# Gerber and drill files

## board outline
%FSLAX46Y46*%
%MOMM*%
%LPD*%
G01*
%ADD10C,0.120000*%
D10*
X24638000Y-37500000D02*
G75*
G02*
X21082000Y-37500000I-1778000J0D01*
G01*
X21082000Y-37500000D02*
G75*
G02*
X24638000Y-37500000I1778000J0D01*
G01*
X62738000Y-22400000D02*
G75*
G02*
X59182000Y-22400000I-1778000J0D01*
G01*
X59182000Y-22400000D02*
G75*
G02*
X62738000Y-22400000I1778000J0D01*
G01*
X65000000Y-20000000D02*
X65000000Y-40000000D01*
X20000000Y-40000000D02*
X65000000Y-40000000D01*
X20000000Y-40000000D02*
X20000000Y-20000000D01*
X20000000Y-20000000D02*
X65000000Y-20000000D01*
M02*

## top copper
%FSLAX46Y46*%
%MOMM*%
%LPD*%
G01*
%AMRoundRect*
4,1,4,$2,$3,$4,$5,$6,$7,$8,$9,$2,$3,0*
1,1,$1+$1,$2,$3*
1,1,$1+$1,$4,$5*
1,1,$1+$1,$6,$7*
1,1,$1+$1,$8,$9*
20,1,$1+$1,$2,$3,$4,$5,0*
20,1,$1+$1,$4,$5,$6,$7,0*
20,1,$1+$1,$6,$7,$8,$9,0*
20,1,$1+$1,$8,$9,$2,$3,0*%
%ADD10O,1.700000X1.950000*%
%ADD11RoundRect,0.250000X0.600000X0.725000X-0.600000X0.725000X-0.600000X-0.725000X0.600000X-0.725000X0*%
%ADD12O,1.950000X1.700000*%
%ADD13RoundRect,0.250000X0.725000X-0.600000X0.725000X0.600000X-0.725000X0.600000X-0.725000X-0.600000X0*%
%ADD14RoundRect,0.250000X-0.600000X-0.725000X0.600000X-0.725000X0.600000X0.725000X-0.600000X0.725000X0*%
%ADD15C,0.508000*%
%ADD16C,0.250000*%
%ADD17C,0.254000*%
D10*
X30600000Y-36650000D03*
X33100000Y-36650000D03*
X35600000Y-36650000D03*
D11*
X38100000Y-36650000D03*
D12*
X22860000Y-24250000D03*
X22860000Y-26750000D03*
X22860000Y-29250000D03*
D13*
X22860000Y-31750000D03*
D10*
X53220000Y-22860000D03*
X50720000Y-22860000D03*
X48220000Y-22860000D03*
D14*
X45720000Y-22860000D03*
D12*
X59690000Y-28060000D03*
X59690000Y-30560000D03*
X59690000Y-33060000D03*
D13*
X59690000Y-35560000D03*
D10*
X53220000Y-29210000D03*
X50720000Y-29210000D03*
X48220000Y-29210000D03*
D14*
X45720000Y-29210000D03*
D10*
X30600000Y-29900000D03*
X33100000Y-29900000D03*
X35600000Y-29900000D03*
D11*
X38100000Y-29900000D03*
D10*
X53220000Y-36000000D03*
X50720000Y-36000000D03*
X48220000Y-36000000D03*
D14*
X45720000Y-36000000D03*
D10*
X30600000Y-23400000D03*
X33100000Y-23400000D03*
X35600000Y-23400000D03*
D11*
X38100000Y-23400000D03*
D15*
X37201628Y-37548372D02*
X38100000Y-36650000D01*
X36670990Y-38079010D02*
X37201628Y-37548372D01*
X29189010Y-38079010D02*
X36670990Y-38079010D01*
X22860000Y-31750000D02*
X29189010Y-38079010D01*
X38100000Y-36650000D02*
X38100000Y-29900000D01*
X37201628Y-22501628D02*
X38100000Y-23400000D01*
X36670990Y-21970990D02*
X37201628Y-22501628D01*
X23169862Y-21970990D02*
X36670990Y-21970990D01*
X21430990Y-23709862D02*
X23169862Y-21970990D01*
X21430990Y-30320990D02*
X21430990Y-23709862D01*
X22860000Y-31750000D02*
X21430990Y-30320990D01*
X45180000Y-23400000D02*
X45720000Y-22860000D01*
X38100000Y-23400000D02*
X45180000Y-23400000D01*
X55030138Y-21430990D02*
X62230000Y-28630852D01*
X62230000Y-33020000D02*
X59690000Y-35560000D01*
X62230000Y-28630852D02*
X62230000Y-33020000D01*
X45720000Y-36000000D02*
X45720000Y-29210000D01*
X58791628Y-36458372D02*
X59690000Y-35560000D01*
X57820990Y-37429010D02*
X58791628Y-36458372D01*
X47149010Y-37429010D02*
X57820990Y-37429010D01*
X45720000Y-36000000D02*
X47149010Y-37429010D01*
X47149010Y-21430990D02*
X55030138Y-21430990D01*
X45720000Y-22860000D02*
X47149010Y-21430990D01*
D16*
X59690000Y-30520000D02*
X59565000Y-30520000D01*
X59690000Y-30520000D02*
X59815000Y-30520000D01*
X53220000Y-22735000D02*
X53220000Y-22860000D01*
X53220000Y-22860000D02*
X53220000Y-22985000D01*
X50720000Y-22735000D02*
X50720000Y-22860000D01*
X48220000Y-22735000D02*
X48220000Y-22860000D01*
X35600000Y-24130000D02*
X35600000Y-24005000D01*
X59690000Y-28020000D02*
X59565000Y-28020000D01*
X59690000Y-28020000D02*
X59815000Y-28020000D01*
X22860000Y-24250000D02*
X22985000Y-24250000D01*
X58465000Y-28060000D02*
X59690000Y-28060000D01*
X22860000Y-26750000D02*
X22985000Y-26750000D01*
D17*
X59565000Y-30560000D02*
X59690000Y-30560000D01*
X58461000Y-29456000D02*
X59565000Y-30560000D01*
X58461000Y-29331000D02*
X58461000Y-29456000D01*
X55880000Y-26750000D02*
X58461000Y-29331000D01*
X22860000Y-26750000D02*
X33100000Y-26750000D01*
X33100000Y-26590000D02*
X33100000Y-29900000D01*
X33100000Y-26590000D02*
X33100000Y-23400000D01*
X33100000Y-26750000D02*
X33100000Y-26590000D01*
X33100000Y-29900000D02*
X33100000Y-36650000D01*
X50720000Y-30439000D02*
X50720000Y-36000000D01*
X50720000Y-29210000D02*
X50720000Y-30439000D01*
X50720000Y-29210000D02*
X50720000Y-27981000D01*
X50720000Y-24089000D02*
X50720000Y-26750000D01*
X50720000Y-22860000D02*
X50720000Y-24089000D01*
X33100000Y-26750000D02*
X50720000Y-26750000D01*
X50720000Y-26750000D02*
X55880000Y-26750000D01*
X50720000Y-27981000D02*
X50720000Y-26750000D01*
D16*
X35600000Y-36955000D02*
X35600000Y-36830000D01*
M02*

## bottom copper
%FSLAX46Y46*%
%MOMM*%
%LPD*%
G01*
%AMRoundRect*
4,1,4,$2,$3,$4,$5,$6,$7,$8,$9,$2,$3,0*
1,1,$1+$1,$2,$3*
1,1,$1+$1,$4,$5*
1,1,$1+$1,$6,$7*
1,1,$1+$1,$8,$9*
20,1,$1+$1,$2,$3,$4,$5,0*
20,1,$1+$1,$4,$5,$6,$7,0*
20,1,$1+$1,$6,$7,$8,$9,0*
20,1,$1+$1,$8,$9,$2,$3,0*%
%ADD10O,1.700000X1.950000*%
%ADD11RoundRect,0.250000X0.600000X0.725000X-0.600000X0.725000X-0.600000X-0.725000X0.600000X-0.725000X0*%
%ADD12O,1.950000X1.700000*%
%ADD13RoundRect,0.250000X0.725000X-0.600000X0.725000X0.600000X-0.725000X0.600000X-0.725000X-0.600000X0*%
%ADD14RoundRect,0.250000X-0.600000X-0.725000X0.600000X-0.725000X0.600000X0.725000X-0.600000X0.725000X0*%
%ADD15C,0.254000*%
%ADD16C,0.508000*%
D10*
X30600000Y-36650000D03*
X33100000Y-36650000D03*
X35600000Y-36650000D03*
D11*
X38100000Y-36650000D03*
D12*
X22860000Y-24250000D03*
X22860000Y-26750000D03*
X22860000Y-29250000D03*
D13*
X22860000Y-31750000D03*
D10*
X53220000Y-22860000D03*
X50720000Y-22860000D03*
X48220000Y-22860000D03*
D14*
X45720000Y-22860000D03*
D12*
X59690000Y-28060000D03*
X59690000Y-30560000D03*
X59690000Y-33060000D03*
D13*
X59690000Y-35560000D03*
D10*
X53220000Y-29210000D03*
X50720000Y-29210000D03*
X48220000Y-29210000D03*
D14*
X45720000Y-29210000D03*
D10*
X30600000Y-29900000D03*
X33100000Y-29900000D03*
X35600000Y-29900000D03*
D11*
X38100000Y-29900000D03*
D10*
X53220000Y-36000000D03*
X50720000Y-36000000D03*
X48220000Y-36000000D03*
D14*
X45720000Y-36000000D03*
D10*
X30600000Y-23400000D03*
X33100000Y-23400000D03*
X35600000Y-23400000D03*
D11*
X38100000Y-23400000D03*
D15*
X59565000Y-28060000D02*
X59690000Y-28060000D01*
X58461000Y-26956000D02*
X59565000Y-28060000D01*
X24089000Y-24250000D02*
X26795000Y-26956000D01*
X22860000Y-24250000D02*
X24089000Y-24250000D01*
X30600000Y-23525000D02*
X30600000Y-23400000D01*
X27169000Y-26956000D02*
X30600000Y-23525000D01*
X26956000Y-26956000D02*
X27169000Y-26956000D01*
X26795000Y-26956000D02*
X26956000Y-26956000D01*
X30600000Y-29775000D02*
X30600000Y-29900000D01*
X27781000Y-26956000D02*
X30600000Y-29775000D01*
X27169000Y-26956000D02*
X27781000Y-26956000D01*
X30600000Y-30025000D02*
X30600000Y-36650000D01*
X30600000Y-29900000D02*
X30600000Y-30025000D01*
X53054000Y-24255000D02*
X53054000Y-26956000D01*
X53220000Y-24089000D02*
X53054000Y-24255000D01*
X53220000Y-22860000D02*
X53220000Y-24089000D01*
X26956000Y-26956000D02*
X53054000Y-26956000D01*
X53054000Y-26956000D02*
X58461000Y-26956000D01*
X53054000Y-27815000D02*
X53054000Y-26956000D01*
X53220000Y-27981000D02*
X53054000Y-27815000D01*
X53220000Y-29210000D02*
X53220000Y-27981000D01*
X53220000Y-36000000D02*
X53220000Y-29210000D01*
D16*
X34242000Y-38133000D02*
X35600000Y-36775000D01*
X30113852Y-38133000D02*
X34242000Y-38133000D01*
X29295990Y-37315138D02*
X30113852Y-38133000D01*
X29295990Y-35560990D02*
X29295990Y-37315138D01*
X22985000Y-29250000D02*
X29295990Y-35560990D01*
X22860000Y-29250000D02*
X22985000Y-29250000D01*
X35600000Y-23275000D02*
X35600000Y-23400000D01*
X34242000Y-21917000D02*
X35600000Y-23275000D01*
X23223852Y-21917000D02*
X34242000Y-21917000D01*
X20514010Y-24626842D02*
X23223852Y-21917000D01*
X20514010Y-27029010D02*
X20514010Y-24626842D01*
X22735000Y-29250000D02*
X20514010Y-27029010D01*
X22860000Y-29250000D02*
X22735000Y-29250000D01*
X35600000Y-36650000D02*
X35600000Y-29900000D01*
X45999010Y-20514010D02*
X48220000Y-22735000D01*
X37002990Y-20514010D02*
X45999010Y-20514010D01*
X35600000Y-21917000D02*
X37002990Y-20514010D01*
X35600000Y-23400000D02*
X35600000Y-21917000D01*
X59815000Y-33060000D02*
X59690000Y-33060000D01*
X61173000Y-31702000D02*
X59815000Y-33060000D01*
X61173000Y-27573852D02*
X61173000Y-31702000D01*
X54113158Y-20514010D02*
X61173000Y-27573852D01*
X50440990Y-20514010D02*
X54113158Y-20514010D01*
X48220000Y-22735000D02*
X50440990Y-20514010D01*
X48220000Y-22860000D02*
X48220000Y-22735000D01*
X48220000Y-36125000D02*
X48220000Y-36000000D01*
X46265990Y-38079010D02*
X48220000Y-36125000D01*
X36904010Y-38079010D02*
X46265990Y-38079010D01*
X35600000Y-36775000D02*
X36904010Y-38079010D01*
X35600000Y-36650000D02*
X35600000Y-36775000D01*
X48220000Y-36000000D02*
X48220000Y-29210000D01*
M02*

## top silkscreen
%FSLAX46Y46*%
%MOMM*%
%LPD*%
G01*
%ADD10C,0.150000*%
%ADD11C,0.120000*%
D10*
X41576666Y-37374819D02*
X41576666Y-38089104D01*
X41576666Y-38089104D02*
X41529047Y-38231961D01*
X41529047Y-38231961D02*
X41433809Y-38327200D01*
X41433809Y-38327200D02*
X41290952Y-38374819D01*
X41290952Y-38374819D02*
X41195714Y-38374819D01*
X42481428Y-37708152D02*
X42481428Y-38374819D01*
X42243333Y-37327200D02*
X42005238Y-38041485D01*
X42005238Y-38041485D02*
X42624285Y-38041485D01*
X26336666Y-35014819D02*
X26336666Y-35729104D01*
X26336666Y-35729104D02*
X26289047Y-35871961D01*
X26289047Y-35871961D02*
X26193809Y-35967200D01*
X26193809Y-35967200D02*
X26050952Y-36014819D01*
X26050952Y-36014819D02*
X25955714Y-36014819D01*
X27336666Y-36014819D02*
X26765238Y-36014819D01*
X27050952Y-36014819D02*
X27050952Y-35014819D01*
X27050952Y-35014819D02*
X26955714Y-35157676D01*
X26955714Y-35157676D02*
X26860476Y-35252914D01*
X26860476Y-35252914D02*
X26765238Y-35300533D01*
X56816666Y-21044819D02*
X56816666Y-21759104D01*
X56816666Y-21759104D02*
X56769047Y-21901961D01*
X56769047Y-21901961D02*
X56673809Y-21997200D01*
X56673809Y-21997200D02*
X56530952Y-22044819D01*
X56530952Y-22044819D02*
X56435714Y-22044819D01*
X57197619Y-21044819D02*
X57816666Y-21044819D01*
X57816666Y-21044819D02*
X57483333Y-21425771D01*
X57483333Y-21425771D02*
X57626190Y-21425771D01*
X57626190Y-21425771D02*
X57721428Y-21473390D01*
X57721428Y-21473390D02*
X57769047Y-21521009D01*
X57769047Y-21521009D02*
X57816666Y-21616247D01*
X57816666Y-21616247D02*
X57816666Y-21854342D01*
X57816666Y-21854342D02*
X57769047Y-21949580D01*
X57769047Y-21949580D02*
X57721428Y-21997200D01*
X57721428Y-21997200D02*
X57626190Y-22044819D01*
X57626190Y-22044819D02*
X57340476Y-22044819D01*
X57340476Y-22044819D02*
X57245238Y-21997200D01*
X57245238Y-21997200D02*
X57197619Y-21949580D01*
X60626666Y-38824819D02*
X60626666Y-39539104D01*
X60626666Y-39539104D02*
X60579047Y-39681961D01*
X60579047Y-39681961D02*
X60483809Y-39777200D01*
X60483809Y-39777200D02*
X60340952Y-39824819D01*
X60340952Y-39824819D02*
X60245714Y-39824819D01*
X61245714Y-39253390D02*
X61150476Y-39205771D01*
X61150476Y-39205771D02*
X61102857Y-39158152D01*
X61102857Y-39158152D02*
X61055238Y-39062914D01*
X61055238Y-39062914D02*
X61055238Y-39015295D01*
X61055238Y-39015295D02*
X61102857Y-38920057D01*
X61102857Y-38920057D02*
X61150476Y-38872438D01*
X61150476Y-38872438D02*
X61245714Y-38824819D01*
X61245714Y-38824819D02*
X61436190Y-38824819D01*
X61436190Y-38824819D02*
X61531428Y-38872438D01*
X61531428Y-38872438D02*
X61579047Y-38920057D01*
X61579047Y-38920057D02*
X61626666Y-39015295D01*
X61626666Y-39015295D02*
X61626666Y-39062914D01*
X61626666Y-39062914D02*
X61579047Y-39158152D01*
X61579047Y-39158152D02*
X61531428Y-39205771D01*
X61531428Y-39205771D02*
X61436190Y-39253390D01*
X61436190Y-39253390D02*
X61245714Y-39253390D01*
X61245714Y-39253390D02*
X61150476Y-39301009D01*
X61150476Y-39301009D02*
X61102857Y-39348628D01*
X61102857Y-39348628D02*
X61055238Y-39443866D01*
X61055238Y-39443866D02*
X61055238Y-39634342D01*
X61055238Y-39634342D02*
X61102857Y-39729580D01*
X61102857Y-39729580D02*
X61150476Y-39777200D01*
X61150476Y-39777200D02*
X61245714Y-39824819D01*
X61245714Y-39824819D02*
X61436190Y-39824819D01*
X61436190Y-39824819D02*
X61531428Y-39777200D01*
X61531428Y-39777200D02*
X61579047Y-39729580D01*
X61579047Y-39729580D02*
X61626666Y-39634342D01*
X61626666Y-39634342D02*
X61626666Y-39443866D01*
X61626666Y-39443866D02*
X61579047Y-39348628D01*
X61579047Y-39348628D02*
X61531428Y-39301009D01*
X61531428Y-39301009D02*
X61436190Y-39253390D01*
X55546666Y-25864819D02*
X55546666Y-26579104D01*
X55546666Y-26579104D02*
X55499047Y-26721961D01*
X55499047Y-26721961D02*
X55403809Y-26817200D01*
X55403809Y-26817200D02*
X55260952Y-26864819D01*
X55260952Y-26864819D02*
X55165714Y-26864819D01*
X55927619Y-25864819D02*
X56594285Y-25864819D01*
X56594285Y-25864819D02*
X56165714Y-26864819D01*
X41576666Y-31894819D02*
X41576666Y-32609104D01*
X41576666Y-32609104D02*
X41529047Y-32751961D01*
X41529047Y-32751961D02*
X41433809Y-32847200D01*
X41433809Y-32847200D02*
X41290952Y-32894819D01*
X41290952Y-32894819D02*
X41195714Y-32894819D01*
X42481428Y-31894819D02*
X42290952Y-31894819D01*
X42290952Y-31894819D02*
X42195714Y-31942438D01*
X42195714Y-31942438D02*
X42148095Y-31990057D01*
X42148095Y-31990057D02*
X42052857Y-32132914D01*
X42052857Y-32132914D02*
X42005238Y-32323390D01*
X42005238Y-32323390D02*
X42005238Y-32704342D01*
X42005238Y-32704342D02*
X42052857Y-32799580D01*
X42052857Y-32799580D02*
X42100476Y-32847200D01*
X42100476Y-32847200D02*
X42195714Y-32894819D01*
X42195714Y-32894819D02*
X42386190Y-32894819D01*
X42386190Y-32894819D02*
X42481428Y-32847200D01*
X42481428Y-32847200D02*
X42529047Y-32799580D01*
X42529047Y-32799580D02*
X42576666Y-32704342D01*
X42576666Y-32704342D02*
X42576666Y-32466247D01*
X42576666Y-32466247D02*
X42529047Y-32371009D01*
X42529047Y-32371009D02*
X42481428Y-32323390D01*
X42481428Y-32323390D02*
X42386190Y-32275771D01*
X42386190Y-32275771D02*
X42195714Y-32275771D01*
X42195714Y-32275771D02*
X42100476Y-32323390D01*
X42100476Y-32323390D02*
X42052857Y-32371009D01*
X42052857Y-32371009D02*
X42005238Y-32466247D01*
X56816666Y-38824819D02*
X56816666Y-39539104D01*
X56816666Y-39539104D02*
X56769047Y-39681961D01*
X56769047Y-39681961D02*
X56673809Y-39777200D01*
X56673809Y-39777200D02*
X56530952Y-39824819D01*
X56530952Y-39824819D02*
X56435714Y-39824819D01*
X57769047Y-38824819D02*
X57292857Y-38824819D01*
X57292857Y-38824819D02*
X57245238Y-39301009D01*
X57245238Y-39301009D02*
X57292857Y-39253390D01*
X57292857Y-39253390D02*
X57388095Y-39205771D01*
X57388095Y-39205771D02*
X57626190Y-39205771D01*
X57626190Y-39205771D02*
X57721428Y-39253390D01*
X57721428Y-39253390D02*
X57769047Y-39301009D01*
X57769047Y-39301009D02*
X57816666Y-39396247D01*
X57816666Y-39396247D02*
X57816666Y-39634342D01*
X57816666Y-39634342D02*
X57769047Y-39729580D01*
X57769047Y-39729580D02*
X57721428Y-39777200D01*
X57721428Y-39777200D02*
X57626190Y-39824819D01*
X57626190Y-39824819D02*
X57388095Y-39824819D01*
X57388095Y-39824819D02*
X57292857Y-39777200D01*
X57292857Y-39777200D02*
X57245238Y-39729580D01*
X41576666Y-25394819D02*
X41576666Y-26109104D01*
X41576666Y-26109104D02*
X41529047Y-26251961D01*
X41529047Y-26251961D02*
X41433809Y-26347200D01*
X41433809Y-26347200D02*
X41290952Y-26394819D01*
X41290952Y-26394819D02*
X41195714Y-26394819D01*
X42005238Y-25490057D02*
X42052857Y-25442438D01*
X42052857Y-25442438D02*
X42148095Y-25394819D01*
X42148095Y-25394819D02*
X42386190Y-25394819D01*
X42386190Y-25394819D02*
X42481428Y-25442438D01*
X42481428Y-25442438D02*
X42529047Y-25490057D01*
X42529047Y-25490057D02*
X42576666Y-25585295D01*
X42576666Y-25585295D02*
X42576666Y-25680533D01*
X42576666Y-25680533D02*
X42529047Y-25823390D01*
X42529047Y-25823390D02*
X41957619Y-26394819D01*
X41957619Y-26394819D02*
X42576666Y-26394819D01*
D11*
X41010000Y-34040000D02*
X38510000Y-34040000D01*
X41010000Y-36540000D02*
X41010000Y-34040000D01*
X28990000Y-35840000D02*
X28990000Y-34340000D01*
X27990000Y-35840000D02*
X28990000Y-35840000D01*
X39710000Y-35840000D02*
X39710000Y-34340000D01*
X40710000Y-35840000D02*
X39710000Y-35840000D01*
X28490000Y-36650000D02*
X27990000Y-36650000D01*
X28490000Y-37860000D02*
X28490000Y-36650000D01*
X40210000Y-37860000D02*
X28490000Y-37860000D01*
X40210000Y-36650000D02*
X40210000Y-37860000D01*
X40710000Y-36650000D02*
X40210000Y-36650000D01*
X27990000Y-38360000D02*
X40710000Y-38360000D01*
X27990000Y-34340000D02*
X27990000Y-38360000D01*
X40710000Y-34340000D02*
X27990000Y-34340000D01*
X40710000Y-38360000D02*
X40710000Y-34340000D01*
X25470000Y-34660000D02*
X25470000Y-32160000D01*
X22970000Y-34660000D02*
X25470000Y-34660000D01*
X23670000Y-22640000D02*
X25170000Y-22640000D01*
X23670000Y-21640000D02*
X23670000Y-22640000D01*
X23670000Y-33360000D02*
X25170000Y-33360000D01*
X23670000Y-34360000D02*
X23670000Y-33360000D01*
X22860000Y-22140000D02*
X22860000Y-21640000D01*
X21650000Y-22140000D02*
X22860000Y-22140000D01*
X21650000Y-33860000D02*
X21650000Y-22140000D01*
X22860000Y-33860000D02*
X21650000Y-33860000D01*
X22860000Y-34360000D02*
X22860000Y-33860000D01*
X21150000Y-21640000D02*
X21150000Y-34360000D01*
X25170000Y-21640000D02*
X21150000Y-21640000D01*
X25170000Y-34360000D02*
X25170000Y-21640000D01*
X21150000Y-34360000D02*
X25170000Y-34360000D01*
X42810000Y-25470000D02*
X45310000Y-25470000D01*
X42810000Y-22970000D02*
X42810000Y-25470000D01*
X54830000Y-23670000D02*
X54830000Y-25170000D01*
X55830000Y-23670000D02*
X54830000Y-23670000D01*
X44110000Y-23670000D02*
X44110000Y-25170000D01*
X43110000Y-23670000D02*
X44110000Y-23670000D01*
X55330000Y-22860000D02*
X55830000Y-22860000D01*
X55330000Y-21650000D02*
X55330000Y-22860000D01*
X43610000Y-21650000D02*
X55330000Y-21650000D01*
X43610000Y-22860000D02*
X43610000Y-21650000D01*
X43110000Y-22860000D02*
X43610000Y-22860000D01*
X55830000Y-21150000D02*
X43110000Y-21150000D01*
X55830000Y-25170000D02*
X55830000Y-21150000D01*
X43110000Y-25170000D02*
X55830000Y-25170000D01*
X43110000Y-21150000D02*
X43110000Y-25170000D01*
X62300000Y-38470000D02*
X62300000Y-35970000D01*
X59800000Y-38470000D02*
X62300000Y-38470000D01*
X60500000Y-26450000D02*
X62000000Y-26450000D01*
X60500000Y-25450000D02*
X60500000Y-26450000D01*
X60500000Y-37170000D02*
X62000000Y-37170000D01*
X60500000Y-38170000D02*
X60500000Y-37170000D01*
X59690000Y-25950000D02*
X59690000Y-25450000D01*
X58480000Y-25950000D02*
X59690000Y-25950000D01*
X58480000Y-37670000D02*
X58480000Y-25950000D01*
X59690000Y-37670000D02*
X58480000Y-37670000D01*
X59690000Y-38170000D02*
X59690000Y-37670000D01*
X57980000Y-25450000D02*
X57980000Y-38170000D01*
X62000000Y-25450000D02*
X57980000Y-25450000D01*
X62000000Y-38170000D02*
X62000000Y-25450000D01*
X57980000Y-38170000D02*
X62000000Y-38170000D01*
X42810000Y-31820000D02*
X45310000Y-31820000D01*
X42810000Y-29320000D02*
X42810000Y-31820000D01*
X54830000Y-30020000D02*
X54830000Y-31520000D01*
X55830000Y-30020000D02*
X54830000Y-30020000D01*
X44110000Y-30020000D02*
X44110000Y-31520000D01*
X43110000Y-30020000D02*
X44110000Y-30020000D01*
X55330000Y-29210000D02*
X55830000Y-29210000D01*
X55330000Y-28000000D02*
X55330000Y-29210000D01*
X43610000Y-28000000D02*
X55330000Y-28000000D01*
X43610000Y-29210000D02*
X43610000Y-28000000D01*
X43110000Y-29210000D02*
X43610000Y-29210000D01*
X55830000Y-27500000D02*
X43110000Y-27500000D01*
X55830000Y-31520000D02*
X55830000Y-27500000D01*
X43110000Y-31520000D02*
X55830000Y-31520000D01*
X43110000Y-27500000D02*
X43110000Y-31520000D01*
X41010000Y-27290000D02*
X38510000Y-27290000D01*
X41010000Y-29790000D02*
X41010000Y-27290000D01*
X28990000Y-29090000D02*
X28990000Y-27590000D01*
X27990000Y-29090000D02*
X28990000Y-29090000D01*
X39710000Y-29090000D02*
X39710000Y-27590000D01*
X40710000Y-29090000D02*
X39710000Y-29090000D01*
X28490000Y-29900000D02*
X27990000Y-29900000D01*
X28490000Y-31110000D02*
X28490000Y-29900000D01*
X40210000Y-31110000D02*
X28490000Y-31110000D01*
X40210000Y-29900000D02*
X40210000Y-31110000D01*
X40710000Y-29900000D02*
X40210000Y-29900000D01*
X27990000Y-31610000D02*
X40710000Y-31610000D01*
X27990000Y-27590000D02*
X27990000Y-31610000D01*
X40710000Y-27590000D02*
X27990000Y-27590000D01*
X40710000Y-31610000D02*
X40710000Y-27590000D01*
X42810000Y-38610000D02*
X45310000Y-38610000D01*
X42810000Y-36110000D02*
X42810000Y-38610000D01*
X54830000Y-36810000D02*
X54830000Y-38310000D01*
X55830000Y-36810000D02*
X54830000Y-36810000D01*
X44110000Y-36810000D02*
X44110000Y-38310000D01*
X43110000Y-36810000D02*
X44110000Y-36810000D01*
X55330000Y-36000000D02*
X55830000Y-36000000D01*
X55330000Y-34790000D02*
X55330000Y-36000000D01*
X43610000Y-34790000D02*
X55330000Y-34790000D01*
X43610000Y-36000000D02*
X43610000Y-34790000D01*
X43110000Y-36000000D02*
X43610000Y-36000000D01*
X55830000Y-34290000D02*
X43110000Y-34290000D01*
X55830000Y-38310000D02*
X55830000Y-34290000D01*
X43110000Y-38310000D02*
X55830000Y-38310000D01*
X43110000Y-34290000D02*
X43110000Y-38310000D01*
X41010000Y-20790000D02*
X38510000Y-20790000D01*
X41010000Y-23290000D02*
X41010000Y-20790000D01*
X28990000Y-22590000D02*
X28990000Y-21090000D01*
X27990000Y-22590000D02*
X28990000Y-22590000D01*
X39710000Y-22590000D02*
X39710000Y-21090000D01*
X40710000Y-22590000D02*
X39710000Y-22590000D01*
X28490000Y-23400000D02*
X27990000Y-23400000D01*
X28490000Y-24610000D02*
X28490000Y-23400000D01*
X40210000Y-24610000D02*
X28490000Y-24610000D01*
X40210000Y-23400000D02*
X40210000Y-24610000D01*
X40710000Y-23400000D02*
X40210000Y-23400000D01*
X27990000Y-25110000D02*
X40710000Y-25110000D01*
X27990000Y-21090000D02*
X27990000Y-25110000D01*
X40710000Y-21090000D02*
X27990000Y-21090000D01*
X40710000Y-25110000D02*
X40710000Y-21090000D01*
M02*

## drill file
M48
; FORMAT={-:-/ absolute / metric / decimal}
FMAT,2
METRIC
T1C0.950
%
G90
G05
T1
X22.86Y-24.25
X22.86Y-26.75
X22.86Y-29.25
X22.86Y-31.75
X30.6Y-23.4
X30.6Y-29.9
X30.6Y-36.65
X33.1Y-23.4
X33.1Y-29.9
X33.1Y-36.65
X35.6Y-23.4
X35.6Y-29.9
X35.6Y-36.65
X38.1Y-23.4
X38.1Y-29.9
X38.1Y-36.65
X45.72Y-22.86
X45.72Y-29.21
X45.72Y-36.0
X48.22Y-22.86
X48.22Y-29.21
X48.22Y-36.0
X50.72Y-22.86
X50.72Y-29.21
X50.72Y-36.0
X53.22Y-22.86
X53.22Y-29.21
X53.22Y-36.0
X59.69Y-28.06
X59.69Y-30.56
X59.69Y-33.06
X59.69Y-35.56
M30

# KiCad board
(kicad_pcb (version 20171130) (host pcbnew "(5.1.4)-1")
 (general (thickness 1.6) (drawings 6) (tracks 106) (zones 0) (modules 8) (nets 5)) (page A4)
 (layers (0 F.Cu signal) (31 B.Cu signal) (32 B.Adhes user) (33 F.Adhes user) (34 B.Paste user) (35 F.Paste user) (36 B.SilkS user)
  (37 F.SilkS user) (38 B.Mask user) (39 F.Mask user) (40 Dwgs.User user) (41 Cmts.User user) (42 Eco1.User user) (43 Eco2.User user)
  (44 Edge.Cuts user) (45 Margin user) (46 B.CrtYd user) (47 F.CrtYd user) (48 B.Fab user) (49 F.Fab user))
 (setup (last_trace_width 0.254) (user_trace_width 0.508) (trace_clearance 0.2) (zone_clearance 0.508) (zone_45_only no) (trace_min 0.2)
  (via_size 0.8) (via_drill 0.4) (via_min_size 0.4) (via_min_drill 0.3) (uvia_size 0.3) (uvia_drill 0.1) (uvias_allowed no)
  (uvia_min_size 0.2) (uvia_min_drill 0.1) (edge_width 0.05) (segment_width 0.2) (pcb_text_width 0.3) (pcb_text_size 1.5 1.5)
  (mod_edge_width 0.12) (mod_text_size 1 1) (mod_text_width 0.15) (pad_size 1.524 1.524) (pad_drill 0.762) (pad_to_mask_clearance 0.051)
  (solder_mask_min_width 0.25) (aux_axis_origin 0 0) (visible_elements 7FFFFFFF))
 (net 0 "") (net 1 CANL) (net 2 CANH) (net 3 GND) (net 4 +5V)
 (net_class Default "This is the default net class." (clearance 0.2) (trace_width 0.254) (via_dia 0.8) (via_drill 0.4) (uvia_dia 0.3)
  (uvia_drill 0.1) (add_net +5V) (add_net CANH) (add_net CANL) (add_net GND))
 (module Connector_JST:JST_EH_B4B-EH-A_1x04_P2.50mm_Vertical (layer F.Cu) (at 38.1 36.65 180)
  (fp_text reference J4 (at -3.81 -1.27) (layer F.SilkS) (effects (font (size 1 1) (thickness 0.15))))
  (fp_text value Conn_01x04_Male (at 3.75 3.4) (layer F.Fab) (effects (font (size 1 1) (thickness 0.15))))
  (fp_line (start -2.91 2.61) (end -0.41 2.61) (layer F.SilkS) (width 0.12))
  (fp_line (start -2.91 0.11) (end -2.91 2.61) (layer F.SilkS) (width 0.12))
  (fp_line (start 9.11 0.81) (end 9.11 2.31) (layer F.SilkS) (width 0.12))
  (fp_line (start 10.11 0.81) (end 9.11 0.81) (layer F.SilkS) (width 0.12))
  (fp_line (start -1.61 0.81) (end -1.61 2.31) (layer F.SilkS) (width 0.12))
  (fp_line (start -2.61 0.81) (end -1.61 0.81) (layer F.SilkS) (width 0.12))
  (fp_line (start 9.61 0) (end 10.11 0) (layer F.SilkS) (width 0.12))
  (fp_line (start 9.61 -1.21) (end 9.61 0) (layer F.SilkS) (width 0.12))
  (fp_line (start -2.11 -1.21) (end 9.61 -1.21) (layer F.SilkS) (width 0.12))
  (fp_line (start -2.11 0) (end -2.11 -1.21) (layer F.SilkS) (width 0.12))
  (fp_line (start -2.61 0) (end -2.11 0) (layer F.SilkS) (width 0.12))
  (fp_line (start 10.11 -1.71) (end -2.61 -1.71) (layer F.SilkS) (width 0.12))
  (fp_line (start 10.11 2.31) (end 10.11 -1.71) (layer F.SilkS) (width 0.12))
  (fp_line (start -2.61 2.31) (end 10.11 2.31) (layer F.SilkS) (width 0.12))
  (fp_line (start -2.61 -1.71) (end -2.61 2.31) (layer F.SilkS) (width 0.12))
  (pad 4 thru_hole oval (at 7.5 0 180) (size 1.7 1.95) (drill 0.95) (layers *.Cu *.Mask) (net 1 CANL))
  (pad 3 thru_hole oval (at 5 0 180) (size 1.7 1.95) (drill 0.95) (layers *.Cu *.Mask) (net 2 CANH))
  (pad 2 thru_hole oval (at 2.5 0 180) (size 1.7 1.95) (drill 0.95) (layers *.Cu *.Mask) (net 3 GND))
  (pad 1 thru_hole roundrect (at 0 0 180) (size 1.7 1.95) (drill 0.95) (layers *.Cu *.Mask) (roundrect_rratio 0.147059) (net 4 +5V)))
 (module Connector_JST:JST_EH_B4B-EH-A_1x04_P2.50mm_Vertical (layer F.Cu) (at 22.86 31.75 90)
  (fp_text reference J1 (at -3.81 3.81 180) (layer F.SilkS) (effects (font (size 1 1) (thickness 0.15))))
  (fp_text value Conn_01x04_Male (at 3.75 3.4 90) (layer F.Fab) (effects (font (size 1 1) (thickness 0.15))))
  (fp_line (start -2.91 2.61) (end -0.41 2.61) (layer F.SilkS) (width 0.12))
  (fp_line (start -2.91 0.11) (end -2.91 2.61) (layer F.SilkS) (width 0.12))
  (fp_line (start 9.11 0.81) (end 9.11 2.31) (layer F.SilkS) (width 0.12))
  (fp_line (start 10.11 0.81) (end 9.11 0.81) (layer F.SilkS) (width 0.12))
  (fp_line (start -1.61 0.81) (end -1.61 2.31) (layer F.SilkS) (width 0.12))
  (fp_line (start -2.61 0.81) (end -1.61 0.81) (layer F.SilkS) (width 0.12))
  (fp_line (start 9.61 0) (end 10.11 0) (layer F.SilkS) (width 0.12))
  (fp_line (start 9.61 -1.21) (end 9.61 0) (layer F.SilkS) (width 0.12))
  (fp_line (start -2.11 -1.21) (end 9.61 -1.21) (layer F.SilkS) (width 0.12))
  (fp_line (start -2.11 0) (end -2.11 -1.21) (layer F.SilkS) (width 0.12))
  (fp_line (start -2.61 0) (end -2.11 0) (layer F.SilkS) (width 0.12))
  (fp_line (start 10.11 -1.71) (end -2.61 -1.71) (layer F.SilkS) (width 0.12))
  (fp_line (start 10.11 2.31) (end 10.11 -1.71) (layer F.SilkS) (width 0.12))
  (fp_line (start -2.61 2.31) (end 10.11 2.31) (layer F.SilkS) (width 0.12))
  (fp_line (start -2.61 -1.71) (end -2.61 2.31) (layer F.SilkS) (width 0.12))
  (pad 4 thru_hole oval (at 7.5 0 90) (size 1.7 1.95) (drill 0.95) (layers *.Cu *.Mask) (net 1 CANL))
  (pad 3 thru_hole oval (at 5 0 90) (size 1.7 1.95) (drill 0.95) (layers *.Cu *.Mask) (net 2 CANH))
  (pad 2 thru_hole oval (at 2.5 0 90) (size 1.7 1.95) (drill 0.95) (layers *.Cu *.Mask) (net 3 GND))
  (pad 1 thru_hole roundrect (at 0 0 90) (size 1.7 1.95) (drill 0.95) (layers *.Cu *.Mask) (roundrect_rratio 0.147059) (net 4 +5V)))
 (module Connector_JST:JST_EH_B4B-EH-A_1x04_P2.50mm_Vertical (layer F.Cu) (at 45.72 22.86)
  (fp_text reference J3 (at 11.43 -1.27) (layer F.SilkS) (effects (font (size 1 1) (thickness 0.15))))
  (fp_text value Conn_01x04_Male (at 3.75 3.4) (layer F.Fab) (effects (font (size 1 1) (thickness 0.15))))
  (fp_line (start -2.91 2.61) (end -0.41 2.61) (layer F.SilkS) (width 0.12))
  (fp_line (start -2.91 0.11) (end -2.91 2.61) (layer F.SilkS) (width 0.12))
  (fp_line (start 9.11 0.81) (end 9.11 2.31) (layer F.SilkS) (width 0.12))
  (fp_line (start 10.11 0.81) (end 9.11 0.81) (layer F.SilkS) (width 0.12))
  (fp_line (start -1.61 0.81) (end -1.61 2.31) (layer F.SilkS) (width 0.12))
  (fp_line (start -2.61 0.81) (end -1.61 0.81) (layer F.SilkS) (width 0.12))
  (fp_line (start 9.61 0) (end 10.11 0) (layer F.SilkS) (width 0.12))
  (fp_line (start 9.61 -1.21) (end 9.61 0) (layer F.SilkS) (width 0.12))
  (fp_line (start -2.11 -1.21) (end 9.61 -1.21) (layer F.SilkS) (width 0.12))
  (fp_line (start -2.11 0) (end -2.11 -1.21) (layer F.SilkS) (width 0.12))
  (fp_line (start -2.61 0) (end -2.11 0) (layer F.SilkS) (width 0.12))
  (fp_line (start 10.11 -1.71) (end -2.61 -1.71) (layer F.SilkS) (width 0.12))
  (fp_line (start 10.11 2.31) (end 10.11 -1.71) (layer F.SilkS) (width 0.12))
  (fp_line (start -2.61 2.31) (end 10.11 2.31) (layer F.SilkS) (width 0.12))
  (fp_line (start -2.61 -1.71) (end -2.61 2.31) (layer F.SilkS) (width 0.12))
  (pad 4 thru_hole oval (at 7.5 0) (size 1.7 1.95) (drill 0.95) (layers *.Cu *.Mask) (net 1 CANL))
  (pad 3 thru_hole oval (at 5 0) (size 1.7 1.95) (drill 0.95) (layers *.Cu *.Mask) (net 2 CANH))
  (pad 2 thru_hole oval (at 2.5 0) (size 1.7 1.95) (drill 0.95) (layers *.Cu *.Mask) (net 3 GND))
  (pad 1 thru_hole roundrect (at 0 0) (size 1.7 1.95) (drill 0.95) (layers *.Cu *.Mask) (roundrect_rratio 0.147059) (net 4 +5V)))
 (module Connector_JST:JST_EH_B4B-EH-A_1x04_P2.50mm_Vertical (layer F.Cu) (at 59.69 35.56 90)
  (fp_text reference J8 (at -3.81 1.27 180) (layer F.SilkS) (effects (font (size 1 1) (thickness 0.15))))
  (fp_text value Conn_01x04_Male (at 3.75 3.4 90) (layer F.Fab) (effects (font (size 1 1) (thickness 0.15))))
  (fp_line (start -2.91 2.61) (end -0.41 2.61) (layer F.SilkS) (width 0.12))
  (fp_line (start -2.91 0.11) (end -2.91 2.61) (layer F.SilkS) (width 0.12))
  (fp_line (start 9.11 0.81) (end 9.11 2.31) (layer F.SilkS) (width 0.12))
  (fp_line (start 10.11 0.81) (end 9.11 0.81) (layer F.SilkS) (width 0.12))
  (fp_line (start -1.61 0.81) (end -1.61 2.31) (layer F.SilkS) (width 0.12))
  (fp_line (start -2.61 0.81) (end -1.61 0.81) (layer F.SilkS) (width 0.12))
  (fp_line (start 9.61 0) (end 10.11 0) (layer F.SilkS) (width 0.12))
  (fp_line (start 9.61 -1.21) (end 9.61 0) (layer F.SilkS) (width 0.12))
  (fp_line (start -2.11 -1.21) (end 9.61 -1.21) (layer F.SilkS) (width 0.12))
  (fp_line (start -2.11 0) (end -2.11 -1.21) (layer F.SilkS) (width 0.12))
  (fp_line (start -2.61 0) (end -2.11 0) (layer F.SilkS) (width 0.12))
  (fp_line (start 10.11 -1.71) (end -2.61 -1.71) (layer F.SilkS) (width 0.12))
  (fp_line (start 10.11 2.31) (end 10.11 -1.71) (layer F.SilkS) (width 0.12))
  (fp_line (start -2.61 2.31) (end 10.11 2.31) (layer F.SilkS) (width 0.12))
  (fp_line (start -2.61 -1.71) (end -2.61 2.31) (layer F.SilkS) (width 0.12))
  (pad 4 thru_hole oval (at 7.5 0 90) (size 1.7 1.95) (drill 0.95) (layers *.Cu *.Mask) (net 1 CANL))
  (pad 3 thru_hole oval (at 5 0 90) (size 1.7 1.95) (drill 0.95) (layers *.Cu *.Mask) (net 2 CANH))
  (pad 2 thru_hole oval (at 2.5 0 90) (size 1.7 1.95) (drill 0.95) (layers *.Cu *.Mask) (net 3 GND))
  (pad 1 thru_hole roundrect (at 0 0 90) (size 1.7 1.95) (drill 0.95) (layers *.Cu *.Mask) (roundrect_rratio 0.147059) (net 4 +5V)))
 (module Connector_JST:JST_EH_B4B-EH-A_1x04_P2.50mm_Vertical (layer F.Cu) (at 45.72 29.21)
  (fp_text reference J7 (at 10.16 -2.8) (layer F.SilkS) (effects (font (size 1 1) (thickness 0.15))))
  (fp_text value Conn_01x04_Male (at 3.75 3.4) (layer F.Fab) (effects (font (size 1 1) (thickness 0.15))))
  (fp_line (start -2.91 2.61) (end -0.41 2.61) (layer F.SilkS) (width 0.12))
  (fp_line (start -2.91 0.11) (end -2.91 2.61) (layer F.SilkS) (width 0.12))
  (fp_line (start 9.11 0.81) (end 9.11 2.31) (layer F.SilkS) (width 0.12))
  (fp_line (start 10.11 0.81) (end 9.11 0.81) (layer F.SilkS) (width 0.12))
  (fp_line (start -1.61 0.81) (end -1.61 2.31) (layer F.SilkS) (width 0.12))
  (fp_line (start -2.61 0.81) (end -1.61 0.81) (layer F.SilkS) (width 0.12))
  (fp_line (start 9.61 0) (end 10.11 0) (layer F.SilkS) (width 0.12))
  (fp_line (start 9.61 -1.21) (end 9.61 0) (layer F.SilkS) (width 0.12))
  (fp_line (start -2.11 -1.21) (end 9.61 -1.21) (layer F.SilkS) (width 0.12))
  (fp_line (start -2.11 0) (end -2.11 -1.21) (layer F.SilkS) (width 0.12))
  (fp_line (start -2.61 0) (end -2.11 0) (layer F.SilkS) (width 0.12))
  (fp_line (start 10.11 -1.71) (end -2.61 -1.71) (layer F.SilkS) (width 0.12))
  (fp_line (start 10.11 2.31) (end 10.11 -1.71) (layer F.SilkS) (width 0.12))
  (fp_line (start -2.61 2.31) (end 10.11 2.31) (layer F.SilkS) (width 0.12))
  (fp_line (start -2.61 -1.71) (end -2.61 2.31) (layer F.SilkS) (width 0.12))
  (pad 4 thru_hole oval (at 7.5 0) (size 1.7 1.95) (drill 0.95) (layers *.Cu *.Mask) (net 1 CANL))
  (pad 3 thru_hole oval (at 5 0) (size 1.7 1.95) (drill 0.95) (layers *.Cu *.Mask) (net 2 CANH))
  (pad 2 thru_hole oval (at 2.5 0) (size 1.7 1.95) (drill 0.95) (layers *.Cu *.Mask) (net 3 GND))
  (pad 1 thru_hole roundrect (at 0 0) (size 1.7 1.95) (drill 0.95) (layers *.Cu *.Mask) (roundrect_rratio 0.147059) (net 4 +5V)))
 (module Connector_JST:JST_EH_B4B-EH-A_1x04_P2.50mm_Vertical (layer F.Cu) (at 38.1 29.9 180)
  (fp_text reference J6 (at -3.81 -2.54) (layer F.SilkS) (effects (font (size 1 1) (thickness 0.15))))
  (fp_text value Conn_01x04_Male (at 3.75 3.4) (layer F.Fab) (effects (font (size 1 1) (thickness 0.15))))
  (fp_line (start -2.91 2.61) (end -0.41 2.61) (layer F.SilkS) (width 0.12))
  (fp_line (start -2.91 0.11) (end -2.91 2.61) (layer F.SilkS) (width 0.12))
  (fp_line (start 9.11 0.81) (end 9.11 2.31) (layer F.SilkS) (width 0.12))
  (fp_line (start 10.11 0.81) (end 9.11 0.81) (layer F.SilkS) (width 0.12))
  (fp_line (start -1.61 0.81) (end -1.61 2.31) (layer F.SilkS) (width 0.12))
  (fp_line (start -2.61 0.81) (end -1.61 0.81) (layer F.SilkS) (width 0.12))
  (fp_line (start 9.61 0) (end 10.11 0) (layer F.SilkS) (width 0.12))
  (fp_line (start 9.61 -1.21) (end 9.61 0) (layer F.SilkS) (width 0.12))
  (fp_line (start -2.11 -1.21) (end 9.61 -1.21) (layer F.SilkS) (width 0.12))
  (fp_line (start -2.11 0) (end -2.11 -1.21) (layer F.SilkS) (width 0.12))
  (fp_line (start -2.61 0) (end -2.11 0) (layer F.SilkS) (width 0.12))
  (fp_line (start 10.11 -1.71) (end -2.61 -1.71) (layer F.SilkS) (width 0.12))
  (fp_line (start 10.11 2.31) (end 10.11 -1.71) (layer F.SilkS) (width 0.12))
  (fp_line (start -2.61 2.31) (end 10.11 2.31) (layer F.SilkS) (width 0.12))
  (fp_line (start -2.61 -1.71) (end -2.61 2.31) (layer F.SilkS) (width 0.12))
  (pad 4 thru_hole oval (at 7.5 0 180) (size 1.7 1.95) (drill 0.95) (layers *.Cu *.Mask) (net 1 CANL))
  (pad 3 thru_hole oval (at 5 0 180) (size 1.7 1.95) (drill 0.95) (layers *.Cu *.Mask) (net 2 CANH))
  (pad 2 thru_hole oval (at 2.5 0 180) (size 1.7 1.95) (drill 0.95) (layers *.Cu *.Mask) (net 3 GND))
  (pad 1 thru_hole roundrect (at 0 0 180) (size 1.7 1.95) (drill 0.95) (layers *.Cu *.Mask) (roundrect_rratio 0.147059) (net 4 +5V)))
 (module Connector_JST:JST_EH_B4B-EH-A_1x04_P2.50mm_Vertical (layer F.Cu) (at 45.72 36)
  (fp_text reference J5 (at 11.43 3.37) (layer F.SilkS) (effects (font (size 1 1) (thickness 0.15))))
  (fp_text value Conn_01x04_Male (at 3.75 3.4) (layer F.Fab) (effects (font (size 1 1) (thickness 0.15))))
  (fp_line (start -2.91 2.61) (end -0.41 2.61) (layer F.SilkS) (width 0.12))
  (fp_line (start -2.91 0.11) (end -2.91 2.61) (layer F.SilkS) (width 0.12))
  (fp_line (start 9.11 0.81) (end 9.11 2.31) (layer F.SilkS) (width 0.12))
  (fp_line (start 10.11 0.81) (end 9.11 0.81) (layer F.SilkS) (width 0.12))
  (fp_line (start -1.61 0.81) (end -1.61 2.31) (layer F.SilkS) (width 0.12))
  (fp_line (start -2.61 0.81) (end -1.61 0.81) (layer F.SilkS) (width 0.12))
  (fp_line (start 9.61 0) (end 10.11 0) (layer F.SilkS) (width 0.12))
  (fp_line (start 9.61 -1.21) (end 9.61 0) (layer F.SilkS) (width 0.12))
  (fp_line (start -2.11 -1.21) (end 9.61 -1.21) (layer F.SilkS) (width 0.12))
  (fp_line (start -2.11 0) (end -2.11 -1.21) (layer F.SilkS) (width 0.12))
  (fp_line (start -2.61 0) (end -2.11 0) (layer F.SilkS) (width 0.12))
  (fp_line (start 10.11 -1.71) (end -2.61 -1.71) (layer F.SilkS) (width 0.12))
  (fp_line (start 10.11 2.31) (end 10.11 -1.71) (layer F.SilkS) (width 0.12))
  (fp_line (start -2.61 2.31) (end 10.11 2.31) (layer F.SilkS) (width 0.12))
  (fp_line (start -2.61 -1.71) (end -2.61 2.31) (layer F.SilkS) (width 0.12))
  (pad 4 thru_hole oval (at 7.5 0) (size 1.7 1.95) (drill 0.95) (layers *.Cu *.Mask) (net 1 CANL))
  (pad 3 thru_hole oval (at 5 0) (size 1.7 1.95) (drill 0.95) (layers *.Cu *.Mask) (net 2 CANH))
  (pad 2 thru_hole oval (at 2.5 0) (size 1.7 1.95) (drill 0.95) (layers *.Cu *.Mask) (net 3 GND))
  (pad 1 thru_hole roundrect (at 0 0) (size 1.7 1.95) (drill 0.95) (layers *.Cu *.Mask) (roundrect_rratio 0.147059) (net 4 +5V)))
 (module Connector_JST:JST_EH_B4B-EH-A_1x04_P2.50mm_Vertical (layer F.Cu) (at 38.1 23.4 180)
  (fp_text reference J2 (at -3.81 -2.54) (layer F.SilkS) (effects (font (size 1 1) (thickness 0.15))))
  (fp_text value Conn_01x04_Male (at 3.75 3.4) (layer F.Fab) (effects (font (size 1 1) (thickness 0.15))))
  (fp_line (start -2.91 2.61) (end -0.41 2.61) (layer F.SilkS) (width 0.12))
  (fp_line (start -2.91 0.11) (end -2.91 2.61) (layer F.SilkS) (width 0.12))
  (fp_line (start 9.11 0.81) (end 9.11 2.31) (layer F.SilkS) (width 0.12))
  (fp_line (start 10.11 0.81) (end 9.11 0.81) (layer F.SilkS) (width 0.12))
  (fp_line (start -1.61 0.81) (end -1.61 2.31) (layer F.SilkS) (width 0.12))
  (fp_line (start -2.61 0.81) (end -1.61 0.81) (layer F.SilkS) (width 0.12))
  (fp_line (start 9.61 0) (end 10.11 0) (layer F.SilkS) (width 0.12))
  (fp_line (start 9.61 -1.21) (end 9.61 0) (layer F.SilkS) (width 0.12))
  (fp_line (start -2.11 -1.21) (end 9.61 -1.21) (layer F.SilkS) (width 0.12))
  (fp_line (start -2.11 0) (end -2.11 -1.21) (layer F.SilkS) (width 0.12))
  (fp_line (start -2.61 0) (end -2.11 0) (layer F.SilkS) (width 0.12))
  (fp_line (start 10.11 -1.71) (end -2.61 -1.71) (layer F.SilkS) (width 0.12))
  (fp_line (start 10.11 2.31) (end 10.11 -1.71) (layer F.SilkS) (width 0.12))
  (fp_line (start -2.61 2.31) (end 10.11 2.31) (layer F.SilkS) (width 0.12))
  (fp_line (start -2.61 -1.71) (end -2.61 2.31) (layer F.SilkS) (width 0.12))
  (pad 4 thru_hole oval (at 7.5 0 180) (size 1.7 1.95) (drill 0.95) (layers *.Cu *.Mask) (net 1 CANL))
  (pad 3 thru_hole oval (at 5 0 180) (size 1.7 1.95) (drill 0.95) (layers *.Cu *.Mask) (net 2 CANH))
  (pad 2 thru_hole oval (at 2.5 0 180) (size 1.7 1.95) (drill 0.95) (layers *.Cu *.Mask) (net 3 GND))
  (pad 1 thru_hole roundrect (at 0 0 180) (size 1.7 1.95) (drill 0.95) (layers *.Cu *.Mask) (roundrect_rratio 0.147059) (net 4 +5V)))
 (gr_circle (center 22.86 37.5) (end 24.638 37.5) (layer Edge.Cuts) (width 0.12))
 (gr_circle (center 60.96 22.4) (end 62.738 22.4) (layer Edge.Cuts) (width 0.12))
 (gr_line (start 65 20) (end 65 40) (layer Edge.Cuts) (width 0.12))
 (gr_line (start 20 40) (end 65 40) (layer Edge.Cuts) (width 0.12))
 (gr_line (start 20 40) (end 20 20) (layer Edge.Cuts) (width 0.12))
 (gr_line (start 20 20) (end 65 20) (layer Edge.Cuts) (width 0.12))
 (segment (start 37.201628 37.548372) (end 38.1 36.65) (width 0.508) (layer F.Cu) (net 4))
 (segment (start 36.67099 38.07901) (end 37.201628 37.548372) (width 0.508) (layer F.Cu) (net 4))
 (segment (start 29.18901 38.07901) (end 36.67099 38.07901) (width 0.508) (layer F.Cu) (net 4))
 (segment (start 22.86 31.75) (end 29.18901 38.07901) (width 0.508) (layer F.Cu) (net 4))
 (segment (start 38.1 36.65) (end 38.1 29.9) (width 0.508) (layer F.Cu) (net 4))
 (segment (start 37.201628 22.501628) (end 38.1 23.4) (width 0.508) (layer F.Cu) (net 4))
 (segment (start 36.67099 21.97099) (end 37.201628 22.501628) (width 0.508) (layer F.Cu) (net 4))
 (segment (start 23.169862 21.97099) (end 36.67099 21.97099) (width 0.508) (layer F.Cu) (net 4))
 (segment (start 21.43099 23.709862) (end 23.169862 21.97099) (width 0.508) (layer F.Cu) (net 4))
 (segment (start 21.43099 30.32099) (end 21.43099 23.709862) (width 0.508) (layer F.Cu) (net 4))
 (segment (start 22.86 31.75) (end 21.43099 30.32099) (width 0.508) (layer F.Cu) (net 4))
 (segment (start 45.18 23.4) (end 45.72 22.86) (width 0.508) (layer F.Cu) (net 4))
 (segment (start 38.1 23.4) (end 45.18 23.4) (width 0.508) (layer F.Cu) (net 4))
 (segment (start 55.030138 21.43099) (end 62.23 28.630852) (width 0.508) (layer F.Cu) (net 4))
 (segment (start 62.23 33.02) (end 59.69 35.56) (width 0.508) (layer F.Cu) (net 4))
 (segment (start 62.23 28.630852) (end 62.23 33.02) (width 0.508) (layer F.Cu) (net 4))
 (segment (start 45.72 36) (end 45.72 29.21) (width 0.508) (layer F.Cu) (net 4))
 (segment (start 58.791628 36.458372) (end 59.69 35.56) (width 0.508) (layer F.Cu) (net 4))
 (segment (start 57.82099 37.42901) (end 58.791628 36.458372) (width 0.508) (layer F.Cu) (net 4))
 (segment (start 47.14901 37.42901) (end 57.82099 37.42901) (width 0.508) (layer F.Cu) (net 4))
 (segment (start 45.72 36) (end 47.14901 37.42901) (width 0.508) (layer F.Cu) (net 4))
 (segment (start 47.14901 21.43099) (end 55.030138 21.43099) (width 0.508) (layer F.Cu) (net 4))
 (segment (start 45.72 22.86) (end 47.14901 21.43099) (width 0.508) (layer F.Cu) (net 4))
 (segment (start 59.69 30.52) (end 59.565 30.52) (width 0.25) (layer F.Cu) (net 2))
 (segment (start 59.69 30.52) (end 59.815 30.52) (width 0.25) (layer F.Cu) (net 2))
 (segment (start 53.22 22.735) (end 53.22 22.86) (width 0.25) (layer F.Cu) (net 1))
 (segment (start 53.22 22.86) (end 53.22 22.985) (width 0.25) (layer F.Cu) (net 1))
 (segment (start 50.72 22.735) (end 50.72 22.86) (width 0.25) (layer F.Cu) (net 2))
 (segment (start 48.22 22.735) (end 48.22 22.86) (width 0.25) (layer F.Cu) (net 3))
 (segment (start 35.6 24.13) (end 35.6 24.005) (width 0.25) (layer F.Cu) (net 3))
 (segment (start 59.69 28.02) (end 59.565 28.02) (width 0.25) (layer F.Cu) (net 1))
 (segment (start 59.69 28.02) (end 59.815 28.02) (width 0.25) (layer F.Cu) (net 1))
 (segment (start 22.86 24.25) (end 22.985 24.25) (width 0.25) (layer F.Cu) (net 1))
 (segment (start 58.465 28.06) (end 59.69 28.06) (width 0.25) (layer F.Cu) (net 1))
 (segment (start 59.565 28.06) (end 59.69 28.06) (width 0.254) (layer B.Cu) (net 1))
 (segment (start 58.461 26.956) (end 59.565 28.06) (width 0.254) (layer B.Cu) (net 1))
 (segment (start 24.089 24.25) (end 26.795 26.956) (width 0.254) (layer B.Cu) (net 1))
 (segment (start 22.86 24.25) (end 24.089 24.25) (width 0.254) (layer B.Cu) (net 1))
 (segment (start 30.6 23.525) (end 30.6 23.4) (width 0.254) (layer B.Cu) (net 1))
 (segment (start 27.169 26.956) (end 30.6 23.525) (width 0.254) (layer B.Cu) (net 1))
 (segment (start 26.956 26.956) (end 27.169 26.956) (width 0.254) (layer B.Cu) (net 1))
 (segment (start 26.795 26.956) (end 26.956 26.956) (width 0.254) (layer B.Cu) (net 1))
 (segment (start 30.6 29.775) (end 30.6 29.9) (width 0.254) (layer B.Cu) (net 1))
 (segment (start 27.781 26.956) (end 30.6 29.775) (width 0.254) (layer B.Cu) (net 1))
 (segment (start 27.169 26.956) (end 27.781 26.956) (width 0.254) (layer B.Cu) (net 1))
 (segment (start 30.6 30.025) (end 30.6 36.65) (width 0.254) (layer B.Cu) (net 1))
 (segment (start 30.6 29.9) (end 30.6 30.025) (width 0.254) (layer B.Cu) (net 1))
 (segment (start 53.054 24.255) (end 53.054 26.956) (width 0.254) (layer B.Cu) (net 1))
 (segment (start 53.22 24.089) (end 53.054 24.255) (width 0.254) (layer B.Cu) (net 1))
 (segment (start 53.22 22.86) (end 53.22 24.089) (width 0.254) (layer B.Cu) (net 1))
 (segment (start 26.956 26.956) (end 53.054 26.956) (width 0.254) (layer B.Cu) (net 1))
 (segment (start 53.054 26.956) (end 58.461 26.956) (width 0.254) (layer B.Cu) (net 1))
 (segment (start 53.054 27.815) (end 53.054 26.956) (width 0.254) (layer B.Cu) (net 1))
 (segment (start 53.22 27.981) (end 53.054 27.815) (width 0.254) (layer B.Cu) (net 1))
 (segment (start 53.22 29.21) (end 53.22 27.981) (width 0.254) (layer B.Cu) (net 1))
 (segment (start 53.22 36) (end 53.22 29.21) (width 0.254) (layer B.Cu) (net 1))
 (segment (start 22.86 26.75) (end 22.985 26.75) (width 0.25) (layer F.Cu) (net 2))
 (segment (start 59.565 30.56) (end 59.69 30.56) (width 0.254) (layer F.Cu) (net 2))
 (segment (start 58.461 29.456) (end 59.565 30.56) (width 0.254) (layer F.Cu) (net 2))
 (segment (start 58.461 29.331) (end 58.461 29.456) (width 0.254) (layer F.Cu) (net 2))
 (segment (start 55.88 26.75) (end 58.461 29.331) (width 0.254) (layer F.Cu) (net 2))
 (segment (start 22.86 26.75) (end 33.1 26.75) (width 0.254) (layer F.Cu) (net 2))
 (segment (start 33.1 26.59) (end 33.1 29.9) (width 0.254) (layer F.Cu) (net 2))
 (segment (start 33.1 26.59) (end 33.1 23.4) (width 0.254) (layer F.Cu) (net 2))
 (segment (start 33.1 26.75) (end 33.1 26.59) (width 0.254) (layer F.Cu) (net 2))
 (segment (start 33.1 29.9) (end 33.1 36.65) (width 0.254) (layer F.Cu) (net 2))
 (segment (start 50.72 30.439) (end 50.72 36) (width 0.254) (layer F.Cu) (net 2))
 (segment (start 50.72 29.21) (end 50.72 30.439) (width 0.254) (layer F.Cu) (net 2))
 (segment (start 50.72 29.21) (end 50.72 27.981) (width 0.254) (layer F.Cu) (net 2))
 (segment (start 50.72 24.089) (end 50.72 26.75) (width 0.254) (layer F.Cu) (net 2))
 (segment (start 50.72 22.86) (end 50.72 24.089) (width 0.254) (layer F.Cu) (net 2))
 (segment (start 33.1 26.75) (end 50.72 26.75) (width 0.254) (layer F.Cu) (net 2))
 (segment (start 50.72 26.75) (end 55.88 26.75) (width 0.254) (layer F.Cu) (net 2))
 (segment (start 50.72 27.981) (end 50.72 26.75) (width 0.254) (layer F.Cu) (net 2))
 (segment (start 35.6 36.955) (end 35.6 36.83) (width 0.25) (layer F.Cu) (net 3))
 (segment (start 34.242 38.133) (end 35.6 36.775) (width 0.508) (layer B.Cu) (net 3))
 (segment (start 30.113852 38.133) (end 34.242 38.133) (width 0.508) (layer B.Cu) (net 3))
 (segment (start 29.29599 37.315138) (end 30.113852 38.133) (width 0.508) (layer B.Cu) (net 3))
 (segment (start 29.29599 35.56099) (end 29.29599 37.315138) (width 0.508) (layer B.Cu) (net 3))
 (segment (start 22.985 29.25) (end 29.29599 35.56099) (width 0.508) (layer B.Cu) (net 3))
 (segment (start 22.86 29.25) (end 22.985 29.25) (width 0.508) (layer B.Cu) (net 3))
 (segment (start 35.6 23.275) (end 35.6 23.4) (width 0.508) (layer B.Cu) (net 3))
 (segment (start 34.242 21.917) (end 35.6 23.275) (width 0.508) (layer B.Cu) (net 3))
 (segment (start 23.223852 21.917) (end 34.242 21.917) (width 0.508) (layer B.Cu) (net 3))
 (segment (start 20.51401 24.626842) (end 23.223852 21.917) (width 0.508) (layer B.Cu) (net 3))
 (segment (start 20.51401 27.02901) (end 20.51401 24.626842) (width 0.508) (layer B.Cu) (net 3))
 (segment (start 22.735 29.25) (end 20.51401 27.02901) (width 0.508) (layer B.Cu) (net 3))
 (segment (start 22.86 29.25) (end 22.735 29.25) (width 0.508) (layer B.Cu) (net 3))
 (segment (start 35.6 36.65) (end 35.6 29.9) (width 0.508) (layer B.Cu) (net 3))
 (segment (start 45.99901 20.51401) (end 48.22 22.735) (width 0.508) (layer B.Cu) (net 3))
 (segment (start 37.00299 20.51401) (end 45.99901 20.51401) (width 0.508) (layer B.Cu) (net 3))
 (segment (start 35.6 21.917) (end 37.00299 20.51401) (width 0.508) (layer B.Cu) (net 3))
 (segment (start 35.6 23.4) (end 35.6 21.917) (width 0.508) (layer B.Cu) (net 3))
 (segment (start 59.815 33.06) (end 59.69 33.06) (width 0.508) (layer B.Cu) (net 3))
 (segment (start 61.173 31.702) (end 59.815 33.06) (width 0.508) (layer B.Cu) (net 3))
 (segment (start 61.173 27.573852) (end 61.173 31.702) (width 0.508) (layer B.Cu) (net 3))
 (segment (start 54.113158 20.51401) (end 61.173 27.573852) (width 0.508) (layer B.Cu) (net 3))
 (segment (start 50.44099 20.51401) (end 54.113158 20.51401) (width 0.508) (layer B.Cu) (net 3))
 (segment (start 48.22 22.735) (end 50.44099 20.51401) (width 0.508) (layer B.Cu) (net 3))
 (segment (start 48.22 22.86) (end 48.22 22.735) (width 0.508) (layer B.Cu) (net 3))
 (segment (start 48.22 36.125) (end 48.22 36) (width 0.508) (layer B.Cu) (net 3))
 (segment (start 46.26599 38.07901) (end 48.22 36.125) (width 0.508) (layer B.Cu) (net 3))
 (segment (start 36.90401 38.07901) (end 46.26599 38.07901) (width 0.508) (layer B.Cu) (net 3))
 (segment (start 35.6 36.775) (end 36.90401 38.07901) (width 0.508) (layer B.Cu) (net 3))
 (segment (start 35.6 36.65) (end 35.6 36.775) (width 0.508) (layer B.Cu) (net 3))
 (segment (start 48.22 36) (end 48.22 29.21) (width 0.508) (layer B.Cu) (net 3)))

